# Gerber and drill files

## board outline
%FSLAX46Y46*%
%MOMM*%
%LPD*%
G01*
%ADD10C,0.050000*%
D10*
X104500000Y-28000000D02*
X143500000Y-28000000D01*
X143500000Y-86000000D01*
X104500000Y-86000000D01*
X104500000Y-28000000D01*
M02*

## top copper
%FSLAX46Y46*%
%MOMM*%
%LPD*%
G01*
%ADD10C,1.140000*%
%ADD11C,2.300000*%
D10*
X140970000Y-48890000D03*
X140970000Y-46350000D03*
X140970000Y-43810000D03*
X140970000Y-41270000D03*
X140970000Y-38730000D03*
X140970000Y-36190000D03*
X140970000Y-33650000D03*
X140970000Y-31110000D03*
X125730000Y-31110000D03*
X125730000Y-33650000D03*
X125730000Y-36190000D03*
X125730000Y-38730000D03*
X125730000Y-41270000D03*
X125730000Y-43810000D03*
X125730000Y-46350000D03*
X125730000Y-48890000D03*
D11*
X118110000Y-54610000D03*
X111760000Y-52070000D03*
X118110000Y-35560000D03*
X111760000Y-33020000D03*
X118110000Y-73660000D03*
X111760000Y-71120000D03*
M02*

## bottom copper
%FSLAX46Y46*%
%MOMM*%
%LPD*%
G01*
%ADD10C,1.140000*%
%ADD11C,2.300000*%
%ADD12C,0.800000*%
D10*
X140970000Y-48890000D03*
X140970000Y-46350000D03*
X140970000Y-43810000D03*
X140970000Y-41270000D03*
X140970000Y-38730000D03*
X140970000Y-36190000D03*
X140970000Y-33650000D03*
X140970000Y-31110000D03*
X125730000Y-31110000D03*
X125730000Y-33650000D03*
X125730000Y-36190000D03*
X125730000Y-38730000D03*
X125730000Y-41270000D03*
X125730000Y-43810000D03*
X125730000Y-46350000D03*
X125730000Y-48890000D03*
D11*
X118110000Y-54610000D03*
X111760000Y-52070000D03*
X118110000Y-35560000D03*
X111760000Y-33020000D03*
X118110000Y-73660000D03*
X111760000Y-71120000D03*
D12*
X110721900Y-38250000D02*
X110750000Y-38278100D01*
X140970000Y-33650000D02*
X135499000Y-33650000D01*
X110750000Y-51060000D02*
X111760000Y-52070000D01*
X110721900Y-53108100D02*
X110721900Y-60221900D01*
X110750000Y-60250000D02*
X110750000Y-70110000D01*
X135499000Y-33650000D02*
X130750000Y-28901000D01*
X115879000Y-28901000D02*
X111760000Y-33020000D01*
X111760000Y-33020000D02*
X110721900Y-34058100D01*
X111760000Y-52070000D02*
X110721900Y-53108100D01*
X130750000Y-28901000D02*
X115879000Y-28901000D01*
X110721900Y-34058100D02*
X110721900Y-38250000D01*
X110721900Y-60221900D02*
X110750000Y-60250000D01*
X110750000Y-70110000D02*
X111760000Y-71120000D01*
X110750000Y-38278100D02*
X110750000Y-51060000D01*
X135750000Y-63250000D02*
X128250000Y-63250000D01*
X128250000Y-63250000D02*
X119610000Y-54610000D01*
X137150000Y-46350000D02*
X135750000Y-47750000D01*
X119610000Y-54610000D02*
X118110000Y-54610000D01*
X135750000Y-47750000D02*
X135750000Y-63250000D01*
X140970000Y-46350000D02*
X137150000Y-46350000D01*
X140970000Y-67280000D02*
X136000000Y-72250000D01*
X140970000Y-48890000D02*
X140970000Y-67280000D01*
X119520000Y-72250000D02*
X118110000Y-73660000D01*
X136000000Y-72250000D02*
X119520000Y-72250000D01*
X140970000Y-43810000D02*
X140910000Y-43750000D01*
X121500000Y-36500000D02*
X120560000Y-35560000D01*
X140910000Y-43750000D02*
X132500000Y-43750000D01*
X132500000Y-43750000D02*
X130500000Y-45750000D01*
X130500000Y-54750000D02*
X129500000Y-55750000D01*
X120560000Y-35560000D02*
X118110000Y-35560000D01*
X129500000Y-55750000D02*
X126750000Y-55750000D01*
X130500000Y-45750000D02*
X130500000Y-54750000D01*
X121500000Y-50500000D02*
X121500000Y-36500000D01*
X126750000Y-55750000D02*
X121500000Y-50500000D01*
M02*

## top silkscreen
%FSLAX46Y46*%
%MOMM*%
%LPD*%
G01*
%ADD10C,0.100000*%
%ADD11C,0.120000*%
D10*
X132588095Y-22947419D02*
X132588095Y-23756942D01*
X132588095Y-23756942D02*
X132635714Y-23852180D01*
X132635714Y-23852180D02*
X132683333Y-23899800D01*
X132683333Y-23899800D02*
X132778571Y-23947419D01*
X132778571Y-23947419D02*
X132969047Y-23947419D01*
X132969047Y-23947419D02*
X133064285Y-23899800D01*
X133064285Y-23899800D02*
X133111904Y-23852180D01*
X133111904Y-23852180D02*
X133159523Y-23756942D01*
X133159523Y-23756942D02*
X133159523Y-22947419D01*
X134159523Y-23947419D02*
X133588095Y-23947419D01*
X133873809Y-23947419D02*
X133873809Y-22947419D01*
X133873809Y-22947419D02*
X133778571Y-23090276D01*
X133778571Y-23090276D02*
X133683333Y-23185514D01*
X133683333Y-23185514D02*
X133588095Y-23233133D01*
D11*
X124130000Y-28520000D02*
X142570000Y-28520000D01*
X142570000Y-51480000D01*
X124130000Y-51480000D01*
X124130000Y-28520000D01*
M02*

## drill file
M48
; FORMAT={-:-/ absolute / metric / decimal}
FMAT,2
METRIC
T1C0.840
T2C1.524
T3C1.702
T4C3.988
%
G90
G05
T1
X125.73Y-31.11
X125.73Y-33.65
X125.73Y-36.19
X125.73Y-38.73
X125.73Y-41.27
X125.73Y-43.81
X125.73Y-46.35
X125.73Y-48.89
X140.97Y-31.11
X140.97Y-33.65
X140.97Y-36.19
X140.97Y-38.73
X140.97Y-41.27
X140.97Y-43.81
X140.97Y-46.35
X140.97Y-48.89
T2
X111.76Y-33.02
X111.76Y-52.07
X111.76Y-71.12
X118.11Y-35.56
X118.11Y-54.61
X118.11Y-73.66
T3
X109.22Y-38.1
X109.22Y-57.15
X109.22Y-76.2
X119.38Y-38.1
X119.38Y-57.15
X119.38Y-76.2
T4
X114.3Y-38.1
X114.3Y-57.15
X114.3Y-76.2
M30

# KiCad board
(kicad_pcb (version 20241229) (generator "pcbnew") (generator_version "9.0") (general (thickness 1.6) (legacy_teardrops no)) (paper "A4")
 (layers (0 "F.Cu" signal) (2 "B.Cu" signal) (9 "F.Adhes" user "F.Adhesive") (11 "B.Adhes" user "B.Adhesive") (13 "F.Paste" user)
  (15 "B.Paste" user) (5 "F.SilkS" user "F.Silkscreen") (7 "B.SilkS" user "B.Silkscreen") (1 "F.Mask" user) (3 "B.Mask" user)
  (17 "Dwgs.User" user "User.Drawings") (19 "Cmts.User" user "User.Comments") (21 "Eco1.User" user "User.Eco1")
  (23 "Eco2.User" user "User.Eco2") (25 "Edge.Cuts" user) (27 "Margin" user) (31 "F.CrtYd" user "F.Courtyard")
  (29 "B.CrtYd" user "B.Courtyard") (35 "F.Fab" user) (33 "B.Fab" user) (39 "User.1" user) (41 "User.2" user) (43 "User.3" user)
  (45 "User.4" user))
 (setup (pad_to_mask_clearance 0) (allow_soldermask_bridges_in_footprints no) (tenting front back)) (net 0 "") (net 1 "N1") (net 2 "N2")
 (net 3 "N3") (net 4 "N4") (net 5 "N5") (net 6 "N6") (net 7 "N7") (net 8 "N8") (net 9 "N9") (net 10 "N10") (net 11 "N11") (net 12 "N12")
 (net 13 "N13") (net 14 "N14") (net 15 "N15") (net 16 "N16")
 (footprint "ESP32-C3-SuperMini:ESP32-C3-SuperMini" (layer "F.Cu") (at 133.35 40)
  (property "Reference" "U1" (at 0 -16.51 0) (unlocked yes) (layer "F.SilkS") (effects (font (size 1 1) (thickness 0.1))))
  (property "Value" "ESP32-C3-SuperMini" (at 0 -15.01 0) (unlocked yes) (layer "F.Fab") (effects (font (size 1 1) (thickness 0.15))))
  (fp_rect (start -9.22 -11.48) (end 9.22 11.48) (stroke (width 0.12) (type solid)) (fill no) (layer "F.SilkS"))
  (pad "1" thru_hole circle (at 7.62 8.89) (size 1.14 1.14) (drill 0.84) (layers "*.Cu" "*.Mask") (remove_unused_layers no) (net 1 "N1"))
  (pad "2" thru_hole circle (at 7.62 6.35) (size 1.14 1.14) (drill 0.84) (layers "*.Cu" "*.Mask") (remove_unused_layers no) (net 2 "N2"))
  (pad "3" thru_hole circle (at 7.62 3.81) (size 1.14 1.14) (drill 0.84) (layers "*.Cu" "*.Mask") (remove_unused_layers no) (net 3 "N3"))
  (pad "4" thru_hole circle (at 7.62 1.27) (size 1.14 1.14) (drill 0.84) (layers "*.Cu" "*.Mask") (remove_unused_layers no) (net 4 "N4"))
  (pad "5" thru_hole circle (at 7.62 -1.27) (size 1.14 1.14) (drill 0.84) (layers "*.Cu" "*.Mask") (remove_unused_layers no) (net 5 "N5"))
  (pad "6" thru_hole circle (at 7.62 -3.81) (size 1.14 1.14) (drill 0.84) (layers "*.Cu" "*.Mask") (remove_unused_layers no) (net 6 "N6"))
  (pad "7" thru_hole circle (at 7.62 -6.35) (size 1.14 1.14) (drill 0.84) (layers "*.Cu" "*.Mask") (remove_unused_layers no) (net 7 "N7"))
  (pad "8" thru_hole circle (at 7.62 -8.89) (size 1.14 1.14) (drill 0.84) (layers "*.Cu" "*.Mask") (remove_unused_layers no) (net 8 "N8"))
  (pad "9" thru_hole circle (at -7.62 -8.89) (size 1.14 1.14) (drill 0.84) (layers "*.Cu" "*.Mask") (remove_unused_layers no) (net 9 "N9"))
  (pad "10" thru_hole circle (at -7.62 -6.35) (size 1.14 1.14) (drill 0.84) (layers "*.Cu" "*.Mask") (remove_unused_layers no)
   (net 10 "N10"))
  (pad "11" thru_hole circle (at -7.62 -3.81) (size 1.14 1.14) (drill 0.84) (layers "*.Cu" "*.Mask") (remove_unused_layers no)
   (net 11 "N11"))
  (pad "12" thru_hole circle (at -7.62 -1.27) (size 1.14 1.14) (drill 0.84) (layers "*.Cu" "*.Mask") (remove_unused_layers no)
   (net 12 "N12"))
  (pad "13" thru_hole circle (at -7.62 1.27) (size 1.14 1.14) (drill 0.84) (layers "*.Cu" "*.Mask") (remove_unused_layers no) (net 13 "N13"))
  (pad "14" thru_hole circle (at -7.62 3.81) (size 1.14 1.14) (drill 0.84) (layers "*.Cu" "*.Mask") (remove_unused_layers no) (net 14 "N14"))
  (pad "15" thru_hole circle (at -7.62 6.35) (size 1.14 1.14) (drill 0.84) (layers "*.Cu" "*.Mask") (remove_unused_layers no) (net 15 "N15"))
  (pad "16" thru_hole circle (at -7.62 8.89) (size 1.14 1.14) (drill 0.84) (layers "*.Cu" "*.Mask") (remove_unused_layers no) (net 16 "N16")))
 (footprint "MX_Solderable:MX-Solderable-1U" (layer "B.Cu") (at 114.3 57.15 180)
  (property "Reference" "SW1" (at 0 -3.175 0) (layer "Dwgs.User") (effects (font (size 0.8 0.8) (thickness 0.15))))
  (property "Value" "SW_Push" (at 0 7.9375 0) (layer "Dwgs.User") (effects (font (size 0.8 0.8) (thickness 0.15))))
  (pad "" np_thru_hole circle (at -5.08 0 131.901) (size 1.7018 1.7018) (drill 1.7018) (layers "*.Cu" "*.Mask"))
  (pad "" np_thru_hole circle (at 0 0 180) (size 3.9878 3.9878) (drill 3.9878) (layers "*.Cu" "*.Mask"))
  (pad "" np_thru_hole circle (at 5.08 0 131.901) (size 1.7018 1.7018) (drill 1.7018) (layers "*.Cu" "*.Mask"))
  (pad "1" thru_hole circle (at -3.81 2.54 180) (size 2.3 2.3) (drill 1.524) (layers "*.Cu" "F.Mask") (remove_unused_layers no) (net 2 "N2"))
  (pad "2" thru_hole circle (at 2.54 5.08 180) (size 2.3 2.3) (drill 1.524) (layers "*.Cu" "F.Mask") (remove_unused_layers no) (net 7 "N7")))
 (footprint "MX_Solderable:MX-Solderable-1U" (layer "B.Cu") (at 114.3 38.1 180)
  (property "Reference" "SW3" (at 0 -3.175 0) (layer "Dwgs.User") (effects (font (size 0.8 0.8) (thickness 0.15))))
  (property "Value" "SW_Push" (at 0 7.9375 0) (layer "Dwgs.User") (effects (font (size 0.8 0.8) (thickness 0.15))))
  (pad "" np_thru_hole circle (at -5.08 0 131.901) (size 1.7018 1.7018) (drill 1.7018) (layers "*.Cu" "*.Mask"))
  (pad "" np_thru_hole circle (at 0 0 180) (size 3.9878 3.9878) (drill 3.9878) (layers "*.Cu" "*.Mask"))
  (pad "" np_thru_hole circle (at 5.08 0 131.901) (size 1.7018 1.7018) (drill 1.7018) (layers "*.Cu" "*.Mask"))
  (pad "1" thru_hole circle (at -3.81 2.54 180) (size 2.3 2.3) (drill 1.524) (layers "*.Cu" "F.Mask") (remove_unused_layers no) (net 3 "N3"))
  (pad "2" thru_hole circle (at 2.54 5.08 180) (size 2.3 2.3) (drill 1.524) (layers "*.Cu" "F.Mask") (remove_unused_layers no) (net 7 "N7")))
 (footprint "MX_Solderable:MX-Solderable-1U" (layer "B.Cu") (at 114.3 76.2 180)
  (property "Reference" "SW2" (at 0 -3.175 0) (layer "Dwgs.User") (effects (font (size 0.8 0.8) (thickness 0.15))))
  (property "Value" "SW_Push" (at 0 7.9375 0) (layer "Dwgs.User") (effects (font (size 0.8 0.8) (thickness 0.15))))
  (pad "" np_thru_hole circle (at -5.08 0 131.901) (size 1.7018 1.7018) (drill 1.7018) (layers "*.Cu" "*.Mask"))
  (pad "" np_thru_hole circle (at 0 0 180) (size 3.9878 3.9878) (drill 3.9878) (layers "*.Cu" "*.Mask"))
  (pad "" np_thru_hole circle (at 5.08 0 131.901) (size 1.7018 1.7018) (drill 1.7018) (layers "*.Cu" "*.Mask"))
  (pad "1" thru_hole circle (at -3.81 2.54 180) (size 2.3 2.3) (drill 1.524) (layers "*.Cu" "F.Mask") (remove_unused_layers no) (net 1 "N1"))
  (pad "2" thru_hole circle (at 2.54 5.08 180) (size 2.3 2.3) (drill 1.524) (layers "*.Cu" "F.Mask") (remove_unused_layers no) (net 7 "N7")))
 (gr_rect (start 104.5 28) (end 143.5 86) (stroke (width 0.05) (type default)) (fill no) (layer "Edge.Cuts"))
 (segment (start 110.7219 38.25) (end 110.75 38.2781) (width 0.8) (layer "B.Cu") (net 7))
 (segment (start 140.97 33.65) (end 135.499 33.65) (width 0.8) (layer "B.Cu") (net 7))
 (segment (start 110.75 51.06) (end 111.76 52.07) (width 0.8) (layer "B.Cu") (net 7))
 (segment (start 110.7219 53.1081) (end 110.7219 60.2219) (width 0.8) (layer "B.Cu") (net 7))
 (segment (start 110.75 60.25) (end 110.75 70.11) (width 0.8) (layer "B.Cu") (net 7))
 (segment (start 135.499 33.65) (end 130.75 28.901) (width 0.8) (layer "B.Cu") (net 7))
 (segment (start 115.879 28.901) (end 111.76 33.02) (width 0.8) (layer "B.Cu") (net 7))
 (segment (start 111.76 33.02) (end 110.7219 34.0581) (width 0.8) (layer "B.Cu") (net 7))
 (segment (start 111.76 52.07) (end 110.7219 53.1081) (width 0.8) (layer "B.Cu") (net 7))
 (segment (start 130.75 28.901) (end 115.879 28.901) (width 0.8) (layer "B.Cu") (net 7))
 (segment (start 110.7219 34.0581) (end 110.7219 38.25) (width 0.8) (layer "B.Cu") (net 7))
 (segment (start 110.7219 60.2219) (end 110.75 60.25) (width 0.8) (layer "B.Cu") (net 7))
 (segment (start 110.75 70.11) (end 111.76 71.12) (width 0.8) (layer "B.Cu") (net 7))
 (segment (start 110.75 38.2781) (end 110.75 51.06) (width 0.8) (layer "B.Cu") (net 7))
 (segment (start 135.75 63.25) (end 128.25 63.25) (width 0.8) (layer "B.Cu") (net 2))
 (segment (start 128.25 63.25) (end 119.61 54.61) (width 0.8) (layer "B.Cu") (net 2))
 (segment (start 137.15 46.35) (end 135.75 47.75) (width 0.8) (layer "B.Cu") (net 2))
 (segment (start 119.61 54.61) (end 118.11 54.61) (width 0.8) (layer "B.Cu") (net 2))
 (segment (start 135.75 47.75) (end 135.75 63.25) (width 0.8) (layer "B.Cu") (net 2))
 (segment (start 140.97 46.35) (end 137.15 46.35) (width 0.8) (layer "B.Cu") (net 2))
 (segment (start 140.97 67.28) (end 136 72.25) (width 0.8) (layer "B.Cu") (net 1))
 (segment (start 140.97 48.89) (end 140.97 67.28) (width 0.8) (layer "B.Cu") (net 1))
 (segment (start 119.52 72.25) (end 118.11 73.66) (width 0.8) (layer "B.Cu") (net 1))
 (segment (start 136 72.25) (end 119.52 72.25) (width 0.8) (layer "B.Cu") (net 1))
 (segment (start 140.97 43.81) (end 140.91 43.75) (width 0.8) (layer "B.Cu") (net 3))
 (segment (start 121.5 36.5) (end 120.56 35.56) (width 0.8) (layer "B.Cu") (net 3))
 (segment (start 140.91 43.75) (end 132.5 43.75) (width 0.8) (layer "B.Cu") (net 3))
 (segment (start 132.5 43.75) (end 130.5 45.75) (width 0.8) (layer "B.Cu") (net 3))
 (segment (start 130.5 54.75) (end 129.5 55.75) (width 0.8) (layer "B.Cu") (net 3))
 (segment (start 120.56 35.56) (end 118.11 35.56) (width 0.8) (layer "B.Cu") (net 3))
 (segment (start 129.5 55.75) (end 126.75 55.75) (width 0.8) (layer "B.Cu") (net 3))
 (segment (start 130.5 45.75) (end 130.5 54.75) (width 0.8) (layer "B.Cu") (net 3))
 (segment (start 121.5 50.5) (end 121.5 36.5) (width 0.8) (layer "B.Cu") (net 3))
 (segment (start 126.75 55.75) (end 121.5 50.5) (width 0.8) (layer "B.Cu") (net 3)))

